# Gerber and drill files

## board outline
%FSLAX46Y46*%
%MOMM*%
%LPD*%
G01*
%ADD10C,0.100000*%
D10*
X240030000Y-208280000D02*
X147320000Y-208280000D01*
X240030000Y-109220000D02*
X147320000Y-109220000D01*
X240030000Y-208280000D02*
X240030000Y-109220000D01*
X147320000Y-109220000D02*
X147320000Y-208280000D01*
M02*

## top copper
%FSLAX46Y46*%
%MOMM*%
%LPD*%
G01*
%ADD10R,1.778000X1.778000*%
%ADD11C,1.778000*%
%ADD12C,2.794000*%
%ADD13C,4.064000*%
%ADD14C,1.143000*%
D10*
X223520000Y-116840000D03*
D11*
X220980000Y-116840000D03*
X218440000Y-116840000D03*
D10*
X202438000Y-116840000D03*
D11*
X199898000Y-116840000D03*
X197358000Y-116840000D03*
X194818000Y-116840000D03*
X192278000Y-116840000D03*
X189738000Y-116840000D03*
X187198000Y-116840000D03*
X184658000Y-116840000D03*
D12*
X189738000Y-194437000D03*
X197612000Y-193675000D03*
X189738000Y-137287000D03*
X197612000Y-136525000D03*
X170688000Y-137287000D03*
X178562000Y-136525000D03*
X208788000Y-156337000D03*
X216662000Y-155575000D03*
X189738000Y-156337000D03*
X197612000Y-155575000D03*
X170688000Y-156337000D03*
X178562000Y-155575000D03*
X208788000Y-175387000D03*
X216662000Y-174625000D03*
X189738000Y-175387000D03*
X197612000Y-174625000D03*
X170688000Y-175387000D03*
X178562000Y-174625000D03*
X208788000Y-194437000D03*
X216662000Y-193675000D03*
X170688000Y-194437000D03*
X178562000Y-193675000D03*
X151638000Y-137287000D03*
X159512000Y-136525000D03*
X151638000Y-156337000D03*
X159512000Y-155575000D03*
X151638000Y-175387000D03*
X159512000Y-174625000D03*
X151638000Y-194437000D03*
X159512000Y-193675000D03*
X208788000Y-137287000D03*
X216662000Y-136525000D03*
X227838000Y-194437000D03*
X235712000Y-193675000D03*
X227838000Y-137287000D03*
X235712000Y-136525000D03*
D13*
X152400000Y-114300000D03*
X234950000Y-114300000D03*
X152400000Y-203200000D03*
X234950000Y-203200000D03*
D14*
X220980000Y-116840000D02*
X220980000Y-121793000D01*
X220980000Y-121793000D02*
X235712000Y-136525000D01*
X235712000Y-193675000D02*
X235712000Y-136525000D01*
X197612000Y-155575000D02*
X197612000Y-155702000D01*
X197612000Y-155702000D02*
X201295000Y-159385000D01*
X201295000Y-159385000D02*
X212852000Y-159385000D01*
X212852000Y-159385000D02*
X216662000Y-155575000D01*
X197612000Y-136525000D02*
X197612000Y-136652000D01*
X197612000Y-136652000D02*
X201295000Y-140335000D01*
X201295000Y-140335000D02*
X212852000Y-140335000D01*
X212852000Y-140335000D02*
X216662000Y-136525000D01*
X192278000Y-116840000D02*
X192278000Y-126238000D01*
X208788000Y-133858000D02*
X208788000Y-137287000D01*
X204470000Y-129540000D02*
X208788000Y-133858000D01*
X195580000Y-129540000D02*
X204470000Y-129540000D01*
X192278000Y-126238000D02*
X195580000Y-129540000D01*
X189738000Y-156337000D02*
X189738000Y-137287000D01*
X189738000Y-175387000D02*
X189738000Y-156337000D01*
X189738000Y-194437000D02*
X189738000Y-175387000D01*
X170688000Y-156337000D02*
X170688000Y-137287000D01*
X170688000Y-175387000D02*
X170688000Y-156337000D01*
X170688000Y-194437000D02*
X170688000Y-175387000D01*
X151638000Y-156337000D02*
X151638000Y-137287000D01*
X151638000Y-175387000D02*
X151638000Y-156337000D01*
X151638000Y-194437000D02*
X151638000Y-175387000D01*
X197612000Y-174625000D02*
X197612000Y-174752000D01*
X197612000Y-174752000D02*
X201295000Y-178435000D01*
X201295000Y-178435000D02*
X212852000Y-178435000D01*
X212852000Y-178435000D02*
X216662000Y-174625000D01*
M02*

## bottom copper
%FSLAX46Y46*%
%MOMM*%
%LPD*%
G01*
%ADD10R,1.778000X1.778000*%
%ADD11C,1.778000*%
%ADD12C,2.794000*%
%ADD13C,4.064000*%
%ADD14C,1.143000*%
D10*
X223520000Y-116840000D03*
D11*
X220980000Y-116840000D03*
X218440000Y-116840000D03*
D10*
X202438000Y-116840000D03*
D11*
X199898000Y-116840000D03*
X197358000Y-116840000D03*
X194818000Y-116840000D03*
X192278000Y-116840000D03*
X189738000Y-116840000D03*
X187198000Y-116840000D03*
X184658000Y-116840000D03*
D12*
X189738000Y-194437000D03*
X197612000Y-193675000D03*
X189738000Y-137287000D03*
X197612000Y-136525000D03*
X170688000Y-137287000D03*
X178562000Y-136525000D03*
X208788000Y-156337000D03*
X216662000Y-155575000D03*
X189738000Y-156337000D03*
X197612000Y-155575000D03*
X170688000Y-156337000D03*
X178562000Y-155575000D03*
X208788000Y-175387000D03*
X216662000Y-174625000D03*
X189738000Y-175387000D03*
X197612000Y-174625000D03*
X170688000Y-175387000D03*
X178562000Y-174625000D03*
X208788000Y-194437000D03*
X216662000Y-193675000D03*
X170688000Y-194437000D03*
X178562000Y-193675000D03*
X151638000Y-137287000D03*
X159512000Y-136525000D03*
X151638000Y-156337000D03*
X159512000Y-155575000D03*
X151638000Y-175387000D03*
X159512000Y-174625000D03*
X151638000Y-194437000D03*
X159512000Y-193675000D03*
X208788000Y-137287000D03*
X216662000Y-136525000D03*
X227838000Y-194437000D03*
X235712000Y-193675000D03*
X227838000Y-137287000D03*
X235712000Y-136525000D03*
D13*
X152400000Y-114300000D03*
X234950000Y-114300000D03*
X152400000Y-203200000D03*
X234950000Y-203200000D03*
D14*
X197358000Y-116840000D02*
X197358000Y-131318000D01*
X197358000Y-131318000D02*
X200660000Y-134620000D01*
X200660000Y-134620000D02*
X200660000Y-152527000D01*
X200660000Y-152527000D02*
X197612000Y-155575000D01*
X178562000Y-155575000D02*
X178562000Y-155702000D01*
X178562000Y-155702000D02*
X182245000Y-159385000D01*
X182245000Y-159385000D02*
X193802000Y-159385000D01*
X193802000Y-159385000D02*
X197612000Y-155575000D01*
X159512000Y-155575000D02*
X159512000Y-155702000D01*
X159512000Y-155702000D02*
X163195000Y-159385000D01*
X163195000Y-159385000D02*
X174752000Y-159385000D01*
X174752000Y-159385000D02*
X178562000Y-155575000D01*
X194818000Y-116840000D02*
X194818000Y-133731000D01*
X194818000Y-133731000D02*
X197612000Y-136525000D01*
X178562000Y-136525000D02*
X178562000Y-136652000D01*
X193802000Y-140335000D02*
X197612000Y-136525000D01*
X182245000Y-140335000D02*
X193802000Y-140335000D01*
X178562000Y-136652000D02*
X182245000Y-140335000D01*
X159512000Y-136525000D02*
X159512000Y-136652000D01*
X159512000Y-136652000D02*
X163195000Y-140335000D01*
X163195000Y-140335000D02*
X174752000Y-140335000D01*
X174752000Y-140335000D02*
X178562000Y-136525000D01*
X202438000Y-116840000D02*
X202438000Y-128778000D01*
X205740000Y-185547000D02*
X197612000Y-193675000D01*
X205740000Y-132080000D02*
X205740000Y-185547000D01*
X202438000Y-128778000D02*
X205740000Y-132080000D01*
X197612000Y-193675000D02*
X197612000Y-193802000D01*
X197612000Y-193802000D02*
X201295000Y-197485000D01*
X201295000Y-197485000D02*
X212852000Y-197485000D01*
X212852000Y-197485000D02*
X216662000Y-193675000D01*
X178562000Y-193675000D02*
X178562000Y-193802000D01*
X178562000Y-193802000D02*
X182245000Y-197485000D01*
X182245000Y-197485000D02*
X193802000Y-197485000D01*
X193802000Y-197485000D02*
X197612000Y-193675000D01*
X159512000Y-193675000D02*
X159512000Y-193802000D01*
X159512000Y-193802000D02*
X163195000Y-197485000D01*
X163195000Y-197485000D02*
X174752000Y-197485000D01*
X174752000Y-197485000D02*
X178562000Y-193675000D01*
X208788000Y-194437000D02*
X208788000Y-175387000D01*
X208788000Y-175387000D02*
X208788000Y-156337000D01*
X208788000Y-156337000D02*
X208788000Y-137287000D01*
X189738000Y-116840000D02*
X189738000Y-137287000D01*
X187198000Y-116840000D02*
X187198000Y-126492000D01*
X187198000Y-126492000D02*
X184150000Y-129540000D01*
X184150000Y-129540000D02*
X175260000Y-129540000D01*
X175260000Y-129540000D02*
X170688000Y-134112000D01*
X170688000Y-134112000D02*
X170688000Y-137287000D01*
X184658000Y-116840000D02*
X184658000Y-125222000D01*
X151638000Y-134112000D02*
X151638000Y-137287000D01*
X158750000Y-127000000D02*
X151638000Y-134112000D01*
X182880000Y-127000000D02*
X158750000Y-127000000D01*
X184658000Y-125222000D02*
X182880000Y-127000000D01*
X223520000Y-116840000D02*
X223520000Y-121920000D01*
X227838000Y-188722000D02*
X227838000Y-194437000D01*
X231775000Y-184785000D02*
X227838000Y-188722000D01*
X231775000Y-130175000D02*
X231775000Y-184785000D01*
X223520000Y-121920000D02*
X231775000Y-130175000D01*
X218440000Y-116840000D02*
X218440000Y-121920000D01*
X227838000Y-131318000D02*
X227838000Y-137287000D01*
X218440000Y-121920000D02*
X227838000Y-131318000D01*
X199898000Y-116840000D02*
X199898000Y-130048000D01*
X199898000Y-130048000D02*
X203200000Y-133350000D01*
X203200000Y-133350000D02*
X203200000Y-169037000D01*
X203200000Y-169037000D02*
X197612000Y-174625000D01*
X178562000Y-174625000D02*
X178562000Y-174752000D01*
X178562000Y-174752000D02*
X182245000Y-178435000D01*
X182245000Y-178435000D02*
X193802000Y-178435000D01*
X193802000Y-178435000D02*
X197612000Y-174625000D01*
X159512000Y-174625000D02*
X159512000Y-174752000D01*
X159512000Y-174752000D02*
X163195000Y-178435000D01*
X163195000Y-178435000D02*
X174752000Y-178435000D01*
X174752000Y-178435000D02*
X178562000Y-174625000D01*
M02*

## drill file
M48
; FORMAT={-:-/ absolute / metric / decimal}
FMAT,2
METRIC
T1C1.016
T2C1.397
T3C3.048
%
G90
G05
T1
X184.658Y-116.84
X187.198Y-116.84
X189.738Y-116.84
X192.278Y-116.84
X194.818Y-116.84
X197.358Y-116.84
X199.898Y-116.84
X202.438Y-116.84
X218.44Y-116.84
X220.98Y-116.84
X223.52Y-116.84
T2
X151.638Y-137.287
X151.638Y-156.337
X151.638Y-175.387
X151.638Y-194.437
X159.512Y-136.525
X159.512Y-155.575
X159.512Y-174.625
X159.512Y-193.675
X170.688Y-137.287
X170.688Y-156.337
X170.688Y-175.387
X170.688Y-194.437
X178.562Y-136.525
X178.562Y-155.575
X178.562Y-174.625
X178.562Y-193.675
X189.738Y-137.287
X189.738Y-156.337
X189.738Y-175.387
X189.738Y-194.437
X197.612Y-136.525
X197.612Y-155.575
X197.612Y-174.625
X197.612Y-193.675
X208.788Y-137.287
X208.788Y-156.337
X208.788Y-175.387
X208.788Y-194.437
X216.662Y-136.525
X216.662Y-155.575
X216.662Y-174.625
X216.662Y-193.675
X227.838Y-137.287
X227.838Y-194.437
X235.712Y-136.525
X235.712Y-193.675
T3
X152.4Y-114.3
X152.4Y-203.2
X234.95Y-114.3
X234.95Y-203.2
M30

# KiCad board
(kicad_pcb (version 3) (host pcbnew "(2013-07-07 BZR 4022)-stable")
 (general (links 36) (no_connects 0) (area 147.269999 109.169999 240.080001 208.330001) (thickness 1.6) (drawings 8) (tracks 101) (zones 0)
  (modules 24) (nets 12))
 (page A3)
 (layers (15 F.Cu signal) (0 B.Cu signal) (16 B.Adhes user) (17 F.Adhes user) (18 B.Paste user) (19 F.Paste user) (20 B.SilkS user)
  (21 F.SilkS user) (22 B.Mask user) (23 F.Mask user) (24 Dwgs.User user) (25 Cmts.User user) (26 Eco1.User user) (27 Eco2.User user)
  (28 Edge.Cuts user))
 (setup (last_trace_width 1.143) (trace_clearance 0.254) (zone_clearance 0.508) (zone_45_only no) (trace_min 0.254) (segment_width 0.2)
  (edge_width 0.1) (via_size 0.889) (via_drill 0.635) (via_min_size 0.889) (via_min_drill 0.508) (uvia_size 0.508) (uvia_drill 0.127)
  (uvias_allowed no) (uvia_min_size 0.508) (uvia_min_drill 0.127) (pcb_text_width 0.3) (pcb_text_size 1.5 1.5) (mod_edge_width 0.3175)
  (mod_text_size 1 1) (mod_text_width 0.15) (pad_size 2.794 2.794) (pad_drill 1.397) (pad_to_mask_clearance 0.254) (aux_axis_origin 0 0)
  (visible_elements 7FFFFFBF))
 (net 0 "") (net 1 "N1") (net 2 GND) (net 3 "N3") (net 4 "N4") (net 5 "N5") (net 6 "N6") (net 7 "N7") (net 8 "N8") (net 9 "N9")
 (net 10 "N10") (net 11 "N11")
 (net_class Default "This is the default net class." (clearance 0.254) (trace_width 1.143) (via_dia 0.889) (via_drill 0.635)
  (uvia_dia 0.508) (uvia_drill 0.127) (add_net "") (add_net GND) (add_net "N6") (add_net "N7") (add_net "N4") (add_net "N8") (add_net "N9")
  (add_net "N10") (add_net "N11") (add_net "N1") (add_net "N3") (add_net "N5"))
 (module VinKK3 (layer F.Cu) (at 214.63 116.84 180)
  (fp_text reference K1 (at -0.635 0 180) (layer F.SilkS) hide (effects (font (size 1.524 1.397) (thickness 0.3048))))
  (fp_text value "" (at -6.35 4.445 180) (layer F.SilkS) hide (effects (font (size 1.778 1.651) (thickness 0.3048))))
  (pad 1 thru_hole rect (at -8.89 0 180) (size 1.778 1.778) (drill 1.016) (layers *.Cu *.Mask F.SilkS) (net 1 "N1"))
  (pad 2 thru_hole circle (at -6.35 0 180) (size 1.778 1.778) (drill 1.016) (layers *.Cu *.Mask F.SilkS) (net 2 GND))
  (pad 3 thru_hole circle (at -3.81 0 180) (size 1.778 1.778) (drill 1.016) (layers *.Cu *.Mask F.SilkS) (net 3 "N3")))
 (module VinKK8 (layer F.Cu) (at 193.548 116.84 180)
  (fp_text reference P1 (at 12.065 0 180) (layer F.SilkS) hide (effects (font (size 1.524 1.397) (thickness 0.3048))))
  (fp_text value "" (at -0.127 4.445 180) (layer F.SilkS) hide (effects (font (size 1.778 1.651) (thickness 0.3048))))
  (pad 1 thru_hole rect (at -8.89 0 180) (size 1.778 1.778) (drill 1.016) (layers *.Cu *.Mask F.SilkS) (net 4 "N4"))
  (pad 2 thru_hole circle (at -6.35 0 180) (size 1.778 1.778) (drill 1.016) (layers *.Cu *.Mask F.SilkS) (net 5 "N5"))
  (pad 3 thru_hole circle (at -3.81 0 180) (size 1.778 1.778) (drill 1.016) (layers *.Cu *.Mask F.SilkS) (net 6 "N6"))
  (pad 4 thru_hole circle (at -1.27 0 180) (size 1.778 1.778) (drill 1.016) (layers *.Cu *.Mask F.SilkS) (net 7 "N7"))
  (pad 5 thru_hole circle (at 1.27 0 180) (size 1.778 1.778) (drill 1.016) (layers *.Cu *.Mask F.SilkS) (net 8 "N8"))
  (pad 6 thru_hole circle (at 3.81 0 180) (size 1.778 1.778) (drill 1.016) (layers *.Cu *.Mask F.SilkS) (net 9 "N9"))
  (pad 7 thru_hole circle (at 6.35 0 180) (size 1.778 1.778) (drill 1.016) (layers *.Cu *.Mask F.SilkS) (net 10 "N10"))
  (pad 8 thru_hole circle (at 8.89 0 180) (size 1.778 1.778) (drill 1.016) (layers *.Cu *.Mask F.SilkS) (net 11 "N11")))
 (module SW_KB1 (layer F.Cu) (at 193.675 189.23)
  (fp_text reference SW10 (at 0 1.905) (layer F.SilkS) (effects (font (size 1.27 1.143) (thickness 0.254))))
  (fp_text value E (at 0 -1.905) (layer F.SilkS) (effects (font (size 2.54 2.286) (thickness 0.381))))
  (pad 1 thru_hole circle (at -3.937 5.207) (size 2.794 2.794) (drill 1.397) (layers *.Cu *.Mask F.SilkS) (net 9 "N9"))
  (pad 2 thru_hole circle (at 3.937 4.445) (size 2.794 2.794) (drill 1.397) (layers *.Cu *.Mask F.SilkS) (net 4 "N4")))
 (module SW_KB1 (layer F.Cu) (at 193.675 132.08)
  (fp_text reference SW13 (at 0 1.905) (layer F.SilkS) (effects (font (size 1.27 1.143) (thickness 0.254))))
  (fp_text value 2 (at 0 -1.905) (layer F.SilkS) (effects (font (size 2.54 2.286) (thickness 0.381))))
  (pad 1 thru_hole circle (at -3.937 5.207) (size 2.794 2.794) (drill 1.397) (layers *.Cu *.Mask F.SilkS) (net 9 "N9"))
  (pad 2 thru_hole circle (at 3.937 4.445) (size 2.794 2.794) (drill 1.397) (layers *.Cu *.Mask F.SilkS) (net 7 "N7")))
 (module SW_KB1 (layer F.Cu) (at 174.625 132.08)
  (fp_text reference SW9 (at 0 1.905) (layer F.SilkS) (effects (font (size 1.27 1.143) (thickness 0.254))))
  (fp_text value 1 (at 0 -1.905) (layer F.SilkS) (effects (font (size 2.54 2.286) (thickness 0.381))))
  (pad 1 thru_hole circle (at -3.937 5.207) (size 2.794 2.794) (drill 1.397) (layers *.Cu *.Mask F.SilkS) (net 10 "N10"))
  (pad 2 thru_hole circle (at 3.937 4.445) (size 2.794 2.794) (drill 1.397) (layers *.Cu *.Mask F.SilkS) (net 7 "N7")))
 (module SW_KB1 (layer F.Cu) (at 212.725 151.13)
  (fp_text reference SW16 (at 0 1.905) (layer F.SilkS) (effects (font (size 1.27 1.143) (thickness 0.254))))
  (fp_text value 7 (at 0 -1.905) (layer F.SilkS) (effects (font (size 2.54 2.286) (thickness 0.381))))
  (pad 1 thru_hole circle (at -3.937 5.207) (size 2.794 2.794) (drill 1.397) (layers *.Cu *.Mask F.SilkS) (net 8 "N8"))
  (pad 2 thru_hole circle (at 3.937 4.445) (size 2.794 2.794) (drill 1.397) (layers *.Cu *.Mask F.SilkS) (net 6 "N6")))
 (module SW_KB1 (layer F.Cu) (at 193.675 151.13)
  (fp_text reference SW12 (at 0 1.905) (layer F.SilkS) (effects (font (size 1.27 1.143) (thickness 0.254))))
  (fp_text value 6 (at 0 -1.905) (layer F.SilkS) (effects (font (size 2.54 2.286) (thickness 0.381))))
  (pad 1 thru_hole circle (at -3.937 5.207) (size 2.794 2.794) (drill 1.397) (layers *.Cu *.Mask F.SilkS) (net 9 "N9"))
  (pad 2 thru_hole circle (at 3.937 4.445) (size 2.794 2.794) (drill 1.397) (layers *.Cu *.Mask F.SilkS) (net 6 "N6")))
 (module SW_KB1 (layer F.Cu) (at 174.625 151.13)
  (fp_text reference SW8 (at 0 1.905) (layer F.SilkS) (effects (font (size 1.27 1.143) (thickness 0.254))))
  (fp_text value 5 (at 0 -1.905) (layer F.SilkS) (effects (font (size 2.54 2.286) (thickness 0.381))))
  (pad 1 thru_hole circle (at -3.937 5.207) (size 2.794 2.794) (drill 1.397) (layers *.Cu *.Mask F.SilkS) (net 10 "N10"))
  (pad 2 thru_hole circle (at 3.937 4.445) (size 2.794 2.794) (drill 1.397) (layers *.Cu *.Mask F.SilkS) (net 6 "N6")))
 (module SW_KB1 (layer F.Cu) (at 212.725 170.18)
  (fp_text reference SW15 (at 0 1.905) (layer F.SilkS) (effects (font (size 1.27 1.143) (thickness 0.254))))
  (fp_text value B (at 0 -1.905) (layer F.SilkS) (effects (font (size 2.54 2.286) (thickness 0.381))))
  (pad 1 thru_hole circle (at -3.937 5.207) (size 2.794 2.794) (drill 1.397) (layers *.Cu *.Mask F.SilkS) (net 8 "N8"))
  (pad 2 thru_hole circle (at 3.937 4.445) (size 2.794 2.794) (drill 1.397) (layers *.Cu *.Mask F.SilkS) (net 5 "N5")))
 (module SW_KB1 (layer F.Cu) (at 193.675 170.18)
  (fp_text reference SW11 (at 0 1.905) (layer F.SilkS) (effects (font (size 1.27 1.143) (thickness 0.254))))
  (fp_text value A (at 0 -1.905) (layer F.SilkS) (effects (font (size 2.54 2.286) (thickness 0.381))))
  (pad 1 thru_hole circle (at -3.937 5.207) (size 2.794 2.794) (drill 1.397) (layers *.Cu *.Mask F.SilkS) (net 9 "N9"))
  (pad 2 thru_hole circle (at 3.937 4.445) (size 2.794 2.794) (drill 1.397) (layers *.Cu *.Mask F.SilkS) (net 5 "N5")))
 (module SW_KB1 (layer F.Cu) (at 174.625 170.18)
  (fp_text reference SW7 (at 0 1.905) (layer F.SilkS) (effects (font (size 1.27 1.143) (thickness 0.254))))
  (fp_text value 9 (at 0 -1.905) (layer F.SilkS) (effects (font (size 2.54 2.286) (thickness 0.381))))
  (pad 1 thru_hole circle (at -3.937 5.207) (size 2.794 2.794) (drill 1.397) (layers *.Cu *.Mask F.SilkS) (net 10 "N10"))
  (pad 2 thru_hole circle (at 3.937 4.445) (size 2.794 2.794) (drill 1.397) (layers *.Cu *.Mask F.SilkS) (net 5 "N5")))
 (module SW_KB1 (layer F.Cu) (at 212.725 189.23)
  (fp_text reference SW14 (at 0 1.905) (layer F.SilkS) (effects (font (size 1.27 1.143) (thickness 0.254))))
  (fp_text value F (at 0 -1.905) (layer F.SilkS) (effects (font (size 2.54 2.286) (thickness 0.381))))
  (pad 1 thru_hole circle (at -3.937 5.207) (size 2.794 2.794) (drill 1.397) (layers *.Cu *.Mask F.SilkS) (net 8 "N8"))
  (pad 2 thru_hole circle (at 3.937 4.445) (size 2.794 2.794) (drill 1.397) (layers *.Cu *.Mask F.SilkS) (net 4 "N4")))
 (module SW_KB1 (layer F.Cu) (at 174.625 189.23)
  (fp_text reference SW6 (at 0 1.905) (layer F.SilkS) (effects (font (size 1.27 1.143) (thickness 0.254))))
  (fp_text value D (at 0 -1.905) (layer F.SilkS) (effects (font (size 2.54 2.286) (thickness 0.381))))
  (pad 1 thru_hole circle (at -3.937 5.207) (size 2.794 2.794) (drill 1.397) (layers *.Cu *.Mask F.SilkS) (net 10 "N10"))
  (pad 2 thru_hole circle (at 3.937 4.445) (size 2.794 2.794) (drill 1.397) (layers *.Cu *.Mask F.SilkS) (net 4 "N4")))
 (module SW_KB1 (layer F.Cu) (at 155.575 132.08)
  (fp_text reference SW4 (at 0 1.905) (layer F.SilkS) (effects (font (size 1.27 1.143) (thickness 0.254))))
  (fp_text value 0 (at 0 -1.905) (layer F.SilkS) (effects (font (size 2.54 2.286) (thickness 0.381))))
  (pad 1 thru_hole circle (at -3.937 5.207) (size 2.794 2.794) (drill 1.397) (layers *.Cu *.Mask F.SilkS) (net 11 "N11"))
  (pad 2 thru_hole circle (at 3.937 4.445) (size 2.794 2.794) (drill 1.397) (layers *.Cu *.Mask F.SilkS) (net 7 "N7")))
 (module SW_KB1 (layer F.Cu) (at 155.575 151.13)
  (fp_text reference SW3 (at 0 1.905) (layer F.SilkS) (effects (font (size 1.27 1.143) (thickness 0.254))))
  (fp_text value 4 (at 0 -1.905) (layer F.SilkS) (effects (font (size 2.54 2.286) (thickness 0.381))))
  (pad 1 thru_hole circle (at -3.937 5.207) (size 2.794 2.794) (drill 1.397) (layers *.Cu *.Mask F.SilkS) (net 11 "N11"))
  (pad 2 thru_hole circle (at 3.937 4.445) (size 2.794 2.794) (drill 1.397) (layers *.Cu *.Mask F.SilkS) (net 6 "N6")))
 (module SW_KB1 (layer F.Cu) (at 155.575 170.18)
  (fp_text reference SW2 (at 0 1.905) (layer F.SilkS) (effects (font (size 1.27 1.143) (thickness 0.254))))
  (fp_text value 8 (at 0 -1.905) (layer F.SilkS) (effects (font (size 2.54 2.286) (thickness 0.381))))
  (pad 1 thru_hole circle (at -3.937 5.207) (size 2.794 2.794) (drill 1.397) (layers *.Cu *.Mask F.SilkS) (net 11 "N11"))
  (pad 2 thru_hole circle (at 3.937 4.445) (size 2.794 2.794) (drill 1.397) (layers *.Cu *.Mask F.SilkS) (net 5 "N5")))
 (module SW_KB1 (layer F.Cu) (at 155.575 189.23)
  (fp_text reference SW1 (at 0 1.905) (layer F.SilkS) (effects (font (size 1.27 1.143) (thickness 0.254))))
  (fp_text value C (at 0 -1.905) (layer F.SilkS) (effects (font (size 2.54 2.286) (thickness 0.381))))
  (pad 1 thru_hole circle (at -3.937 5.207) (size 2.794 2.794) (drill 1.397) (layers *.Cu *.Mask F.SilkS) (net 11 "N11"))
  (pad 2 thru_hole circle (at 3.937 4.445) (size 2.794 2.794) (drill 1.397) (layers *.Cu *.Mask F.SilkS) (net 4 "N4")))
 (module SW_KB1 (layer F.Cu) (at 212.725 132.08)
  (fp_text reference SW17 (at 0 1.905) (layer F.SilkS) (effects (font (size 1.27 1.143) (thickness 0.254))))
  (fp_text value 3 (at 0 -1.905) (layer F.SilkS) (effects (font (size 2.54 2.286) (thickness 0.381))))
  (pad 1 thru_hole circle (at -3.937 5.207) (size 2.794 2.794) (drill 1.397) (layers *.Cu *.Mask F.SilkS) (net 8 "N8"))
  (pad 2 thru_hole circle (at 3.937 4.445) (size 2.794 2.794) (drill 1.397) (layers *.Cu *.Mask F.SilkS) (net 7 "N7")))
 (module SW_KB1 (layer F.Cu) (at 231.775 189.23)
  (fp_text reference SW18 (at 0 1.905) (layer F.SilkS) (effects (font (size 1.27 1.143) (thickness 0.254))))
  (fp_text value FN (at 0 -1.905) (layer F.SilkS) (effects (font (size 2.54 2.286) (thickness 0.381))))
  (pad 1 thru_hole circle (at -3.937 5.207) (size 2.794 2.794) (drill 1.397) (layers *.Cu *.Mask F.SilkS) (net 1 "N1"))
  (pad 2 thru_hole circle (at 3.937 4.445) (size 2.794 2.794) (drill 1.397) (layers *.Cu *.Mask F.SilkS) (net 2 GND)))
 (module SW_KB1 (layer F.Cu) (at 231.775 132.08)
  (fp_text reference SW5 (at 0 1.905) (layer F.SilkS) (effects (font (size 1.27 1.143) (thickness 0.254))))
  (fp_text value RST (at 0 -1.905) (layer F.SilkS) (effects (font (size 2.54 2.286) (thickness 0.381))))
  (pad 1 thru_hole circle (at -3.937 5.207) (size 2.794 2.794) (drill 1.397) (layers *.Cu *.Mask F.SilkS) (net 3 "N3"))
  (pad 2 thru_hole circle (at 3.937 4.445) (size 2.794 2.794) (drill 1.397) (layers *.Cu *.Mask F.SilkS) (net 2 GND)))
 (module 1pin (layer F.Cu) (at 152.4 114.3)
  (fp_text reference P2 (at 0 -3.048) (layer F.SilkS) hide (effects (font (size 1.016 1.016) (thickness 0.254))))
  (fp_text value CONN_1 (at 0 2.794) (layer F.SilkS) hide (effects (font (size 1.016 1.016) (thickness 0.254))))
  (pad 1 thru_hole circle (at 0 0) (size 4.064 4.064) (drill 3.048) (layers *.Cu *.Mask F.SilkS)))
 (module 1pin (layer F.Cu) (at 234.95 114.3)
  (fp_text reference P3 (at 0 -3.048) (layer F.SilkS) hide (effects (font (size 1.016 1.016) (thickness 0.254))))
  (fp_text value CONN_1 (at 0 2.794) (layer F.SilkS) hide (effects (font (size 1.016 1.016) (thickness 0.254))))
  (pad 1 thru_hole circle (at 0 0) (size 4.064 4.064) (drill 3.048) (layers *.Cu *.Mask F.SilkS)))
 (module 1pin (layer F.Cu) (at 152.4 203.2)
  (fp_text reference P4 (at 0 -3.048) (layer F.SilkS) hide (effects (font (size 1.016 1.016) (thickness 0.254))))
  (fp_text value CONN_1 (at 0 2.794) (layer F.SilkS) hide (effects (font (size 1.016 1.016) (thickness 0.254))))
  (pad 1 thru_hole circle (at 0 0) (size 4.064 4.064) (drill 3.048) (layers *.Cu *.Mask F.SilkS)))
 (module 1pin (layer F.Cu) (at 234.95 203.2)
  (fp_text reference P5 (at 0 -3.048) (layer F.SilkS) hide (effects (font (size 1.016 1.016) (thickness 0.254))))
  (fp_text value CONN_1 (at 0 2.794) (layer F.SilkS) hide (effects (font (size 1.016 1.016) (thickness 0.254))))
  (pad 1 thru_hole circle (at 0 0) (size 4.064 4.064) (drill 3.048) (layers *.Cu *.Mask F.SilkS)))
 (gr_line (start 240.03 208.28) (end 147.32 208.28) (angle 90) (layer Edge.Cuts) (width 0.1))
 (gr_line (start 240.03 109.22) (end 147.32 109.22) (angle 90) (layer Edge.Cuts) (width 0.1))
 (gr_line (start 240.03 208.28) (end 240.03 109.22) (angle 90) (layer Edge.Cuts) (width 0.1))
 (gr_line (start 147.32 109.22) (end 147.32 208.28) (angle 90) (layer Edge.Cuts) (width 0.1))
 (segment (start 220.98 116.84) (end 220.98 121.793) (width 1.143) (layer F.Cu) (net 2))
 (segment (start 220.98 121.793) (end 235.712 136.525) (width 1.143) (layer F.Cu) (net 2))
 (segment (start 235.712 193.675) (end 235.712 136.525) (width 1.143) (layer F.Cu) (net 2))
 (segment (start 197.612 155.575) (end 197.612 155.702) (width 1.143) (layer F.Cu) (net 6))
 (segment (start 197.612 155.702) (end 201.295 159.385) (width 1.143) (layer F.Cu) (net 6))
 (segment (start 201.295 159.385) (end 212.852 159.385) (width 1.143) (layer F.Cu) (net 6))
 (segment (start 212.852 159.385) (end 216.662 155.575) (width 1.143) (layer F.Cu) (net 6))
 (segment (start 197.358 116.84) (end 197.358 131.318) (width 1.143) (layer B.Cu) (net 6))
 (segment (start 197.358 131.318) (end 200.66 134.62) (width 1.143) (layer B.Cu) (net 6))
 (segment (start 200.66 134.62) (end 200.66 152.527) (width 1.143) (layer B.Cu) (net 6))
 (segment (start 200.66 152.527) (end 197.612 155.575) (width 1.143) (layer B.Cu) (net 6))
 (segment (start 178.562 155.575) (end 178.562 155.702) (width 1.143) (layer B.Cu) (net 6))
 (segment (start 178.562 155.702) (end 182.245 159.385) (width 1.143) (layer B.Cu) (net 6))
 (segment (start 182.245 159.385) (end 193.802 159.385) (width 1.143) (layer B.Cu) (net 6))
 (segment (start 193.802 159.385) (end 197.612 155.575) (width 1.143) (layer B.Cu) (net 6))
 (segment (start 159.512 155.575) (end 159.512 155.702) (width 1.143) (layer B.Cu) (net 6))
 (segment (start 159.512 155.702) (end 163.195 159.385) (width 1.143) (layer B.Cu) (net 6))
 (segment (start 163.195 159.385) (end 174.752 159.385) (width 1.143) (layer B.Cu) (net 6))
 (segment (start 174.752 159.385) (end 178.562 155.575) (width 1.143) (layer B.Cu) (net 6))
 (segment (start 197.612 136.525) (end 197.612 136.652) (width 1.143) (layer F.Cu) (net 7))
 (segment (start 197.612 136.652) (end 201.295 140.335) (width 1.143) (layer F.Cu) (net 7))
 (segment (start 201.295 140.335) (end 212.852 140.335) (width 1.143) (layer F.Cu) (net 7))
 (segment (start 212.852 140.335) (end 216.662 136.525) (width 1.143) (layer F.Cu) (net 7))
 (segment (start 194.818 116.84) (end 194.818 133.731) (width 1.143) (layer B.Cu) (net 7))
 (segment (start 194.818 133.731) (end 197.612 136.525) (width 1.143) (layer B.Cu) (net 7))
 (segment (start 178.562 136.525) (end 178.562 136.652) (width 1.143) (layer B.Cu) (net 7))
 (segment (start 193.802 140.335) (end 197.612 136.525) (width 1.143) (layer B.Cu) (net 7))
 (segment (start 182.245 140.335) (end 193.802 140.335) (width 1.143) (layer B.Cu) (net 7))
 (segment (start 178.562 136.652) (end 182.245 140.335) (width 1.143) (layer B.Cu) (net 7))
 (segment (start 159.512 136.525) (end 159.512 136.652) (width 1.143) (layer B.Cu) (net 7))
 (segment (start 159.512 136.652) (end 163.195 140.335) (width 1.143) (layer B.Cu) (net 7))
 (segment (start 163.195 140.335) (end 174.752 140.335) (width 1.143) (layer B.Cu) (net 7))
 (segment (start 174.752 140.335) (end 178.562 136.525) (width 1.143) (layer B.Cu) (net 7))
 (segment (start 202.438 116.84) (end 202.438 128.778) (width 1.143) (layer B.Cu) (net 4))
 (segment (start 205.74 185.547) (end 197.612 193.675) (width 1.143) (layer B.Cu) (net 4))
 (segment (start 205.74 132.08) (end 205.74 185.547) (width 1.143) (layer B.Cu) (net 4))
 (segment (start 202.438 128.778) (end 205.74 132.08) (width 1.143) (layer B.Cu) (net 4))
 (segment (start 197.612 193.675) (end 197.612 193.802) (width 1.143) (layer B.Cu) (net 4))
 (segment (start 197.612 193.802) (end 201.295 197.485) (width 1.143) (layer B.Cu) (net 4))
 (segment (start 201.295 197.485) (end 212.852 197.485) (width 1.143) (layer B.Cu) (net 4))
 (segment (start 212.852 197.485) (end 216.662 193.675) (width 1.143) (layer B.Cu) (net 4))
 (segment (start 178.562 193.675) (end 178.562 193.802) (width 1.143) (layer B.Cu) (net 4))
 (segment (start 178.562 193.802) (end 182.245 197.485) (width 1.143) (layer B.Cu) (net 4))
 (segment (start 182.245 197.485) (end 193.802 197.485) (width 1.143) (layer B.Cu) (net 4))
 (segment (start 193.802 197.485) (end 197.612 193.675) (width 1.143) (layer B.Cu) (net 4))
 (segment (start 159.512 193.675) (end 159.512 193.802) (width 1.143) (layer B.Cu) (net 4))
 (segment (start 159.512 193.802) (end 163.195 197.485) (width 1.143) (layer B.Cu) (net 4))
 (segment (start 163.195 197.485) (end 174.752 197.485) (width 1.143) (layer B.Cu) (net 4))
 (segment (start 174.752 197.485) (end 178.562 193.675) (width 1.143) (layer B.Cu) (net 4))
 (segment (start 208.788 194.437) (end 208.788 175.387) (width 1.143) (layer B.Cu) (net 8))
 (segment (start 208.788 175.387) (end 208.788 156.337) (width 1.143) (layer B.Cu) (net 8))
 (segment (start 208.788 156.337) (end 208.788 137.287) (width 1.143) (layer B.Cu) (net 8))
 (segment (start 192.278 116.84) (end 192.278 126.238) (width 1.143) (layer F.Cu) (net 8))
 (segment (start 208.788 133.858) (end 208.788 137.287) (width 1.143) (layer F.Cu) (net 8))
 (segment (start 204.47 129.54) (end 208.788 133.858) (width 1.143) (layer F.Cu) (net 8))
 (segment (start 195.58 129.54) (end 204.47 129.54) (width 1.143) (layer F.Cu) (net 8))
 (segment (start 192.278 126.238) (end 195.58 129.54) (width 1.143) (layer F.Cu) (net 8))
 (segment (start 189.738 116.84) (end 189.738 137.287) (width 1.143) (layer B.Cu) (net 9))
 (segment (start 189.738 156.337) (end 189.738 137.287) (width 1.143) (layer F.Cu) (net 9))
 (segment (start 189.738 175.387) (end 189.738 156.337) (width 1.143) (layer F.Cu) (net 9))
 (segment (start 189.738 194.437) (end 189.738 175.387) (width 1.143) (layer F.Cu) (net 9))
 (segment (start 187.198 116.84) (end 187.198 126.492) (width 1.143) (layer B.Cu) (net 10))
 (segment (start 187.198 126.492) (end 184.15 129.54) (width 1.143) (layer B.Cu) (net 10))
 (segment (start 184.15 129.54) (end 175.26 129.54) (width 1.143) (layer B.Cu) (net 10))
 (segment (start 175.26 129.54) (end 170.688 134.112) (width 1.143) (layer B.Cu) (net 10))
 (segment (start 170.688 134.112) (end 170.688 137.287) (width 1.143) (layer B.Cu) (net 10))
 (segment (start 170.688 156.337) (end 170.688 137.287) (width 1.143) (layer F.Cu) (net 10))
 (segment (start 170.688 175.387) (end 170.688 156.337) (width 1.143) (layer F.Cu) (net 10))
 (segment (start 170.688 194.437) (end 170.688 175.387) (width 1.143) (layer F.Cu) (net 10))
 (segment (start 184.658 116.84) (end 184.658 125.222) (width 1.143) (layer B.Cu) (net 11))
 (segment (start 151.638 134.112) (end 151.638 137.287) (width 1.143) (layer B.Cu) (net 11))
 (segment (start 158.75 127) (end 151.638 134.112) (width 1.143) (layer B.Cu) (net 11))
 (segment (start 182.88 127) (end 158.75 127) (width 1.143) (layer B.Cu) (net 11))
 (segment (start 184.658 125.222) (end 182.88 127) (width 1.143) (layer B.Cu) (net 11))
 (segment (start 151.638 156.337) (end 151.638 137.287) (width 1.143) (layer F.Cu) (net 11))
 (segment (start 151.638 175.387) (end 151.638 156.337) (width 1.143) (layer F.Cu) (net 11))
 (segment (start 151.638 194.437) (end 151.638 175.387) (width 1.143) (layer F.Cu) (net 11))
 (segment (start 223.52 116.84) (end 223.52 121.92) (width 1.143) (layer B.Cu) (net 1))
 (segment (start 227.838 188.722) (end 227.838 194.437) (width 1.143) (layer B.Cu) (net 1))
 (segment (start 231.775 184.785) (end 227.838 188.722) (width 1.143) (layer B.Cu) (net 1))
 (segment (start 231.775 130.175) (end 231.775 184.785) (width 1.143) (layer B.Cu) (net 1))
 (segment (start 223.52 121.92) (end 231.775 130.175) (width 1.143) (layer B.Cu) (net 1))
 (segment (start 218.44 116.84) (end 218.44 121.92) (width 1.143) (layer B.Cu) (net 3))
 (segment (start 227.838 131.318) (end 227.838 137.287) (width 1.143) (layer B.Cu) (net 3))
 (segment (start 218.44 121.92) (end 227.838 131.318) (width 1.143) (layer B.Cu) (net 3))
 (segment (start 197.612 174.625) (end 197.612 174.752) (width 1.143) (layer F.Cu) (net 5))
 (segment (start 197.612 174.752) (end 201.295 178.435) (width 1.143) (layer F.Cu) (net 5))
 (segment (start 201.295 178.435) (end 212.852 178.435) (width 1.143) (layer F.Cu) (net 5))
 (segment (start 212.852 178.435) (end 216.662 174.625) (width 1.143) (layer F.Cu) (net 5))
 (segment (start 199.898 116.84) (end 199.898 130.048) (width 1.143) (layer B.Cu) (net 5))
 (segment (start 199.898 130.048) (end 203.2 133.35) (width 1.143) (layer B.Cu) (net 5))
 (segment (start 203.2 133.35) (end 203.2 169.037) (width 1.143) (layer B.Cu) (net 5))
 (segment (start 203.2 169.037) (end 197.612 174.625) (width 1.143) (layer B.Cu) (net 5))
 (segment (start 178.562 174.625) (end 178.562 174.752) (width 1.143) (layer B.Cu) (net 5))
 (segment (start 178.562 174.752) (end 182.245 178.435) (width 1.143) (layer B.Cu) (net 5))
 (segment (start 182.245 178.435) (end 193.802 178.435) (width 1.143) (layer B.Cu) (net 5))
 (segment (start 193.802 178.435) (end 197.612 174.625) (width 1.143) (layer B.Cu) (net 5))
 (segment (start 159.512 174.625) (end 159.512 174.752) (width 1.143) (layer B.Cu) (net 5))
 (segment (start 159.512 174.752) (end 163.195 178.435) (width 1.143) (layer B.Cu) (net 5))
 (segment (start 163.195 178.435) (end 174.752 178.435) (width 1.143) (layer B.Cu) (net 5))
 (segment (start 174.752 178.435) (end 178.562 174.625) (width 1.143) (layer B.Cu) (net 5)))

